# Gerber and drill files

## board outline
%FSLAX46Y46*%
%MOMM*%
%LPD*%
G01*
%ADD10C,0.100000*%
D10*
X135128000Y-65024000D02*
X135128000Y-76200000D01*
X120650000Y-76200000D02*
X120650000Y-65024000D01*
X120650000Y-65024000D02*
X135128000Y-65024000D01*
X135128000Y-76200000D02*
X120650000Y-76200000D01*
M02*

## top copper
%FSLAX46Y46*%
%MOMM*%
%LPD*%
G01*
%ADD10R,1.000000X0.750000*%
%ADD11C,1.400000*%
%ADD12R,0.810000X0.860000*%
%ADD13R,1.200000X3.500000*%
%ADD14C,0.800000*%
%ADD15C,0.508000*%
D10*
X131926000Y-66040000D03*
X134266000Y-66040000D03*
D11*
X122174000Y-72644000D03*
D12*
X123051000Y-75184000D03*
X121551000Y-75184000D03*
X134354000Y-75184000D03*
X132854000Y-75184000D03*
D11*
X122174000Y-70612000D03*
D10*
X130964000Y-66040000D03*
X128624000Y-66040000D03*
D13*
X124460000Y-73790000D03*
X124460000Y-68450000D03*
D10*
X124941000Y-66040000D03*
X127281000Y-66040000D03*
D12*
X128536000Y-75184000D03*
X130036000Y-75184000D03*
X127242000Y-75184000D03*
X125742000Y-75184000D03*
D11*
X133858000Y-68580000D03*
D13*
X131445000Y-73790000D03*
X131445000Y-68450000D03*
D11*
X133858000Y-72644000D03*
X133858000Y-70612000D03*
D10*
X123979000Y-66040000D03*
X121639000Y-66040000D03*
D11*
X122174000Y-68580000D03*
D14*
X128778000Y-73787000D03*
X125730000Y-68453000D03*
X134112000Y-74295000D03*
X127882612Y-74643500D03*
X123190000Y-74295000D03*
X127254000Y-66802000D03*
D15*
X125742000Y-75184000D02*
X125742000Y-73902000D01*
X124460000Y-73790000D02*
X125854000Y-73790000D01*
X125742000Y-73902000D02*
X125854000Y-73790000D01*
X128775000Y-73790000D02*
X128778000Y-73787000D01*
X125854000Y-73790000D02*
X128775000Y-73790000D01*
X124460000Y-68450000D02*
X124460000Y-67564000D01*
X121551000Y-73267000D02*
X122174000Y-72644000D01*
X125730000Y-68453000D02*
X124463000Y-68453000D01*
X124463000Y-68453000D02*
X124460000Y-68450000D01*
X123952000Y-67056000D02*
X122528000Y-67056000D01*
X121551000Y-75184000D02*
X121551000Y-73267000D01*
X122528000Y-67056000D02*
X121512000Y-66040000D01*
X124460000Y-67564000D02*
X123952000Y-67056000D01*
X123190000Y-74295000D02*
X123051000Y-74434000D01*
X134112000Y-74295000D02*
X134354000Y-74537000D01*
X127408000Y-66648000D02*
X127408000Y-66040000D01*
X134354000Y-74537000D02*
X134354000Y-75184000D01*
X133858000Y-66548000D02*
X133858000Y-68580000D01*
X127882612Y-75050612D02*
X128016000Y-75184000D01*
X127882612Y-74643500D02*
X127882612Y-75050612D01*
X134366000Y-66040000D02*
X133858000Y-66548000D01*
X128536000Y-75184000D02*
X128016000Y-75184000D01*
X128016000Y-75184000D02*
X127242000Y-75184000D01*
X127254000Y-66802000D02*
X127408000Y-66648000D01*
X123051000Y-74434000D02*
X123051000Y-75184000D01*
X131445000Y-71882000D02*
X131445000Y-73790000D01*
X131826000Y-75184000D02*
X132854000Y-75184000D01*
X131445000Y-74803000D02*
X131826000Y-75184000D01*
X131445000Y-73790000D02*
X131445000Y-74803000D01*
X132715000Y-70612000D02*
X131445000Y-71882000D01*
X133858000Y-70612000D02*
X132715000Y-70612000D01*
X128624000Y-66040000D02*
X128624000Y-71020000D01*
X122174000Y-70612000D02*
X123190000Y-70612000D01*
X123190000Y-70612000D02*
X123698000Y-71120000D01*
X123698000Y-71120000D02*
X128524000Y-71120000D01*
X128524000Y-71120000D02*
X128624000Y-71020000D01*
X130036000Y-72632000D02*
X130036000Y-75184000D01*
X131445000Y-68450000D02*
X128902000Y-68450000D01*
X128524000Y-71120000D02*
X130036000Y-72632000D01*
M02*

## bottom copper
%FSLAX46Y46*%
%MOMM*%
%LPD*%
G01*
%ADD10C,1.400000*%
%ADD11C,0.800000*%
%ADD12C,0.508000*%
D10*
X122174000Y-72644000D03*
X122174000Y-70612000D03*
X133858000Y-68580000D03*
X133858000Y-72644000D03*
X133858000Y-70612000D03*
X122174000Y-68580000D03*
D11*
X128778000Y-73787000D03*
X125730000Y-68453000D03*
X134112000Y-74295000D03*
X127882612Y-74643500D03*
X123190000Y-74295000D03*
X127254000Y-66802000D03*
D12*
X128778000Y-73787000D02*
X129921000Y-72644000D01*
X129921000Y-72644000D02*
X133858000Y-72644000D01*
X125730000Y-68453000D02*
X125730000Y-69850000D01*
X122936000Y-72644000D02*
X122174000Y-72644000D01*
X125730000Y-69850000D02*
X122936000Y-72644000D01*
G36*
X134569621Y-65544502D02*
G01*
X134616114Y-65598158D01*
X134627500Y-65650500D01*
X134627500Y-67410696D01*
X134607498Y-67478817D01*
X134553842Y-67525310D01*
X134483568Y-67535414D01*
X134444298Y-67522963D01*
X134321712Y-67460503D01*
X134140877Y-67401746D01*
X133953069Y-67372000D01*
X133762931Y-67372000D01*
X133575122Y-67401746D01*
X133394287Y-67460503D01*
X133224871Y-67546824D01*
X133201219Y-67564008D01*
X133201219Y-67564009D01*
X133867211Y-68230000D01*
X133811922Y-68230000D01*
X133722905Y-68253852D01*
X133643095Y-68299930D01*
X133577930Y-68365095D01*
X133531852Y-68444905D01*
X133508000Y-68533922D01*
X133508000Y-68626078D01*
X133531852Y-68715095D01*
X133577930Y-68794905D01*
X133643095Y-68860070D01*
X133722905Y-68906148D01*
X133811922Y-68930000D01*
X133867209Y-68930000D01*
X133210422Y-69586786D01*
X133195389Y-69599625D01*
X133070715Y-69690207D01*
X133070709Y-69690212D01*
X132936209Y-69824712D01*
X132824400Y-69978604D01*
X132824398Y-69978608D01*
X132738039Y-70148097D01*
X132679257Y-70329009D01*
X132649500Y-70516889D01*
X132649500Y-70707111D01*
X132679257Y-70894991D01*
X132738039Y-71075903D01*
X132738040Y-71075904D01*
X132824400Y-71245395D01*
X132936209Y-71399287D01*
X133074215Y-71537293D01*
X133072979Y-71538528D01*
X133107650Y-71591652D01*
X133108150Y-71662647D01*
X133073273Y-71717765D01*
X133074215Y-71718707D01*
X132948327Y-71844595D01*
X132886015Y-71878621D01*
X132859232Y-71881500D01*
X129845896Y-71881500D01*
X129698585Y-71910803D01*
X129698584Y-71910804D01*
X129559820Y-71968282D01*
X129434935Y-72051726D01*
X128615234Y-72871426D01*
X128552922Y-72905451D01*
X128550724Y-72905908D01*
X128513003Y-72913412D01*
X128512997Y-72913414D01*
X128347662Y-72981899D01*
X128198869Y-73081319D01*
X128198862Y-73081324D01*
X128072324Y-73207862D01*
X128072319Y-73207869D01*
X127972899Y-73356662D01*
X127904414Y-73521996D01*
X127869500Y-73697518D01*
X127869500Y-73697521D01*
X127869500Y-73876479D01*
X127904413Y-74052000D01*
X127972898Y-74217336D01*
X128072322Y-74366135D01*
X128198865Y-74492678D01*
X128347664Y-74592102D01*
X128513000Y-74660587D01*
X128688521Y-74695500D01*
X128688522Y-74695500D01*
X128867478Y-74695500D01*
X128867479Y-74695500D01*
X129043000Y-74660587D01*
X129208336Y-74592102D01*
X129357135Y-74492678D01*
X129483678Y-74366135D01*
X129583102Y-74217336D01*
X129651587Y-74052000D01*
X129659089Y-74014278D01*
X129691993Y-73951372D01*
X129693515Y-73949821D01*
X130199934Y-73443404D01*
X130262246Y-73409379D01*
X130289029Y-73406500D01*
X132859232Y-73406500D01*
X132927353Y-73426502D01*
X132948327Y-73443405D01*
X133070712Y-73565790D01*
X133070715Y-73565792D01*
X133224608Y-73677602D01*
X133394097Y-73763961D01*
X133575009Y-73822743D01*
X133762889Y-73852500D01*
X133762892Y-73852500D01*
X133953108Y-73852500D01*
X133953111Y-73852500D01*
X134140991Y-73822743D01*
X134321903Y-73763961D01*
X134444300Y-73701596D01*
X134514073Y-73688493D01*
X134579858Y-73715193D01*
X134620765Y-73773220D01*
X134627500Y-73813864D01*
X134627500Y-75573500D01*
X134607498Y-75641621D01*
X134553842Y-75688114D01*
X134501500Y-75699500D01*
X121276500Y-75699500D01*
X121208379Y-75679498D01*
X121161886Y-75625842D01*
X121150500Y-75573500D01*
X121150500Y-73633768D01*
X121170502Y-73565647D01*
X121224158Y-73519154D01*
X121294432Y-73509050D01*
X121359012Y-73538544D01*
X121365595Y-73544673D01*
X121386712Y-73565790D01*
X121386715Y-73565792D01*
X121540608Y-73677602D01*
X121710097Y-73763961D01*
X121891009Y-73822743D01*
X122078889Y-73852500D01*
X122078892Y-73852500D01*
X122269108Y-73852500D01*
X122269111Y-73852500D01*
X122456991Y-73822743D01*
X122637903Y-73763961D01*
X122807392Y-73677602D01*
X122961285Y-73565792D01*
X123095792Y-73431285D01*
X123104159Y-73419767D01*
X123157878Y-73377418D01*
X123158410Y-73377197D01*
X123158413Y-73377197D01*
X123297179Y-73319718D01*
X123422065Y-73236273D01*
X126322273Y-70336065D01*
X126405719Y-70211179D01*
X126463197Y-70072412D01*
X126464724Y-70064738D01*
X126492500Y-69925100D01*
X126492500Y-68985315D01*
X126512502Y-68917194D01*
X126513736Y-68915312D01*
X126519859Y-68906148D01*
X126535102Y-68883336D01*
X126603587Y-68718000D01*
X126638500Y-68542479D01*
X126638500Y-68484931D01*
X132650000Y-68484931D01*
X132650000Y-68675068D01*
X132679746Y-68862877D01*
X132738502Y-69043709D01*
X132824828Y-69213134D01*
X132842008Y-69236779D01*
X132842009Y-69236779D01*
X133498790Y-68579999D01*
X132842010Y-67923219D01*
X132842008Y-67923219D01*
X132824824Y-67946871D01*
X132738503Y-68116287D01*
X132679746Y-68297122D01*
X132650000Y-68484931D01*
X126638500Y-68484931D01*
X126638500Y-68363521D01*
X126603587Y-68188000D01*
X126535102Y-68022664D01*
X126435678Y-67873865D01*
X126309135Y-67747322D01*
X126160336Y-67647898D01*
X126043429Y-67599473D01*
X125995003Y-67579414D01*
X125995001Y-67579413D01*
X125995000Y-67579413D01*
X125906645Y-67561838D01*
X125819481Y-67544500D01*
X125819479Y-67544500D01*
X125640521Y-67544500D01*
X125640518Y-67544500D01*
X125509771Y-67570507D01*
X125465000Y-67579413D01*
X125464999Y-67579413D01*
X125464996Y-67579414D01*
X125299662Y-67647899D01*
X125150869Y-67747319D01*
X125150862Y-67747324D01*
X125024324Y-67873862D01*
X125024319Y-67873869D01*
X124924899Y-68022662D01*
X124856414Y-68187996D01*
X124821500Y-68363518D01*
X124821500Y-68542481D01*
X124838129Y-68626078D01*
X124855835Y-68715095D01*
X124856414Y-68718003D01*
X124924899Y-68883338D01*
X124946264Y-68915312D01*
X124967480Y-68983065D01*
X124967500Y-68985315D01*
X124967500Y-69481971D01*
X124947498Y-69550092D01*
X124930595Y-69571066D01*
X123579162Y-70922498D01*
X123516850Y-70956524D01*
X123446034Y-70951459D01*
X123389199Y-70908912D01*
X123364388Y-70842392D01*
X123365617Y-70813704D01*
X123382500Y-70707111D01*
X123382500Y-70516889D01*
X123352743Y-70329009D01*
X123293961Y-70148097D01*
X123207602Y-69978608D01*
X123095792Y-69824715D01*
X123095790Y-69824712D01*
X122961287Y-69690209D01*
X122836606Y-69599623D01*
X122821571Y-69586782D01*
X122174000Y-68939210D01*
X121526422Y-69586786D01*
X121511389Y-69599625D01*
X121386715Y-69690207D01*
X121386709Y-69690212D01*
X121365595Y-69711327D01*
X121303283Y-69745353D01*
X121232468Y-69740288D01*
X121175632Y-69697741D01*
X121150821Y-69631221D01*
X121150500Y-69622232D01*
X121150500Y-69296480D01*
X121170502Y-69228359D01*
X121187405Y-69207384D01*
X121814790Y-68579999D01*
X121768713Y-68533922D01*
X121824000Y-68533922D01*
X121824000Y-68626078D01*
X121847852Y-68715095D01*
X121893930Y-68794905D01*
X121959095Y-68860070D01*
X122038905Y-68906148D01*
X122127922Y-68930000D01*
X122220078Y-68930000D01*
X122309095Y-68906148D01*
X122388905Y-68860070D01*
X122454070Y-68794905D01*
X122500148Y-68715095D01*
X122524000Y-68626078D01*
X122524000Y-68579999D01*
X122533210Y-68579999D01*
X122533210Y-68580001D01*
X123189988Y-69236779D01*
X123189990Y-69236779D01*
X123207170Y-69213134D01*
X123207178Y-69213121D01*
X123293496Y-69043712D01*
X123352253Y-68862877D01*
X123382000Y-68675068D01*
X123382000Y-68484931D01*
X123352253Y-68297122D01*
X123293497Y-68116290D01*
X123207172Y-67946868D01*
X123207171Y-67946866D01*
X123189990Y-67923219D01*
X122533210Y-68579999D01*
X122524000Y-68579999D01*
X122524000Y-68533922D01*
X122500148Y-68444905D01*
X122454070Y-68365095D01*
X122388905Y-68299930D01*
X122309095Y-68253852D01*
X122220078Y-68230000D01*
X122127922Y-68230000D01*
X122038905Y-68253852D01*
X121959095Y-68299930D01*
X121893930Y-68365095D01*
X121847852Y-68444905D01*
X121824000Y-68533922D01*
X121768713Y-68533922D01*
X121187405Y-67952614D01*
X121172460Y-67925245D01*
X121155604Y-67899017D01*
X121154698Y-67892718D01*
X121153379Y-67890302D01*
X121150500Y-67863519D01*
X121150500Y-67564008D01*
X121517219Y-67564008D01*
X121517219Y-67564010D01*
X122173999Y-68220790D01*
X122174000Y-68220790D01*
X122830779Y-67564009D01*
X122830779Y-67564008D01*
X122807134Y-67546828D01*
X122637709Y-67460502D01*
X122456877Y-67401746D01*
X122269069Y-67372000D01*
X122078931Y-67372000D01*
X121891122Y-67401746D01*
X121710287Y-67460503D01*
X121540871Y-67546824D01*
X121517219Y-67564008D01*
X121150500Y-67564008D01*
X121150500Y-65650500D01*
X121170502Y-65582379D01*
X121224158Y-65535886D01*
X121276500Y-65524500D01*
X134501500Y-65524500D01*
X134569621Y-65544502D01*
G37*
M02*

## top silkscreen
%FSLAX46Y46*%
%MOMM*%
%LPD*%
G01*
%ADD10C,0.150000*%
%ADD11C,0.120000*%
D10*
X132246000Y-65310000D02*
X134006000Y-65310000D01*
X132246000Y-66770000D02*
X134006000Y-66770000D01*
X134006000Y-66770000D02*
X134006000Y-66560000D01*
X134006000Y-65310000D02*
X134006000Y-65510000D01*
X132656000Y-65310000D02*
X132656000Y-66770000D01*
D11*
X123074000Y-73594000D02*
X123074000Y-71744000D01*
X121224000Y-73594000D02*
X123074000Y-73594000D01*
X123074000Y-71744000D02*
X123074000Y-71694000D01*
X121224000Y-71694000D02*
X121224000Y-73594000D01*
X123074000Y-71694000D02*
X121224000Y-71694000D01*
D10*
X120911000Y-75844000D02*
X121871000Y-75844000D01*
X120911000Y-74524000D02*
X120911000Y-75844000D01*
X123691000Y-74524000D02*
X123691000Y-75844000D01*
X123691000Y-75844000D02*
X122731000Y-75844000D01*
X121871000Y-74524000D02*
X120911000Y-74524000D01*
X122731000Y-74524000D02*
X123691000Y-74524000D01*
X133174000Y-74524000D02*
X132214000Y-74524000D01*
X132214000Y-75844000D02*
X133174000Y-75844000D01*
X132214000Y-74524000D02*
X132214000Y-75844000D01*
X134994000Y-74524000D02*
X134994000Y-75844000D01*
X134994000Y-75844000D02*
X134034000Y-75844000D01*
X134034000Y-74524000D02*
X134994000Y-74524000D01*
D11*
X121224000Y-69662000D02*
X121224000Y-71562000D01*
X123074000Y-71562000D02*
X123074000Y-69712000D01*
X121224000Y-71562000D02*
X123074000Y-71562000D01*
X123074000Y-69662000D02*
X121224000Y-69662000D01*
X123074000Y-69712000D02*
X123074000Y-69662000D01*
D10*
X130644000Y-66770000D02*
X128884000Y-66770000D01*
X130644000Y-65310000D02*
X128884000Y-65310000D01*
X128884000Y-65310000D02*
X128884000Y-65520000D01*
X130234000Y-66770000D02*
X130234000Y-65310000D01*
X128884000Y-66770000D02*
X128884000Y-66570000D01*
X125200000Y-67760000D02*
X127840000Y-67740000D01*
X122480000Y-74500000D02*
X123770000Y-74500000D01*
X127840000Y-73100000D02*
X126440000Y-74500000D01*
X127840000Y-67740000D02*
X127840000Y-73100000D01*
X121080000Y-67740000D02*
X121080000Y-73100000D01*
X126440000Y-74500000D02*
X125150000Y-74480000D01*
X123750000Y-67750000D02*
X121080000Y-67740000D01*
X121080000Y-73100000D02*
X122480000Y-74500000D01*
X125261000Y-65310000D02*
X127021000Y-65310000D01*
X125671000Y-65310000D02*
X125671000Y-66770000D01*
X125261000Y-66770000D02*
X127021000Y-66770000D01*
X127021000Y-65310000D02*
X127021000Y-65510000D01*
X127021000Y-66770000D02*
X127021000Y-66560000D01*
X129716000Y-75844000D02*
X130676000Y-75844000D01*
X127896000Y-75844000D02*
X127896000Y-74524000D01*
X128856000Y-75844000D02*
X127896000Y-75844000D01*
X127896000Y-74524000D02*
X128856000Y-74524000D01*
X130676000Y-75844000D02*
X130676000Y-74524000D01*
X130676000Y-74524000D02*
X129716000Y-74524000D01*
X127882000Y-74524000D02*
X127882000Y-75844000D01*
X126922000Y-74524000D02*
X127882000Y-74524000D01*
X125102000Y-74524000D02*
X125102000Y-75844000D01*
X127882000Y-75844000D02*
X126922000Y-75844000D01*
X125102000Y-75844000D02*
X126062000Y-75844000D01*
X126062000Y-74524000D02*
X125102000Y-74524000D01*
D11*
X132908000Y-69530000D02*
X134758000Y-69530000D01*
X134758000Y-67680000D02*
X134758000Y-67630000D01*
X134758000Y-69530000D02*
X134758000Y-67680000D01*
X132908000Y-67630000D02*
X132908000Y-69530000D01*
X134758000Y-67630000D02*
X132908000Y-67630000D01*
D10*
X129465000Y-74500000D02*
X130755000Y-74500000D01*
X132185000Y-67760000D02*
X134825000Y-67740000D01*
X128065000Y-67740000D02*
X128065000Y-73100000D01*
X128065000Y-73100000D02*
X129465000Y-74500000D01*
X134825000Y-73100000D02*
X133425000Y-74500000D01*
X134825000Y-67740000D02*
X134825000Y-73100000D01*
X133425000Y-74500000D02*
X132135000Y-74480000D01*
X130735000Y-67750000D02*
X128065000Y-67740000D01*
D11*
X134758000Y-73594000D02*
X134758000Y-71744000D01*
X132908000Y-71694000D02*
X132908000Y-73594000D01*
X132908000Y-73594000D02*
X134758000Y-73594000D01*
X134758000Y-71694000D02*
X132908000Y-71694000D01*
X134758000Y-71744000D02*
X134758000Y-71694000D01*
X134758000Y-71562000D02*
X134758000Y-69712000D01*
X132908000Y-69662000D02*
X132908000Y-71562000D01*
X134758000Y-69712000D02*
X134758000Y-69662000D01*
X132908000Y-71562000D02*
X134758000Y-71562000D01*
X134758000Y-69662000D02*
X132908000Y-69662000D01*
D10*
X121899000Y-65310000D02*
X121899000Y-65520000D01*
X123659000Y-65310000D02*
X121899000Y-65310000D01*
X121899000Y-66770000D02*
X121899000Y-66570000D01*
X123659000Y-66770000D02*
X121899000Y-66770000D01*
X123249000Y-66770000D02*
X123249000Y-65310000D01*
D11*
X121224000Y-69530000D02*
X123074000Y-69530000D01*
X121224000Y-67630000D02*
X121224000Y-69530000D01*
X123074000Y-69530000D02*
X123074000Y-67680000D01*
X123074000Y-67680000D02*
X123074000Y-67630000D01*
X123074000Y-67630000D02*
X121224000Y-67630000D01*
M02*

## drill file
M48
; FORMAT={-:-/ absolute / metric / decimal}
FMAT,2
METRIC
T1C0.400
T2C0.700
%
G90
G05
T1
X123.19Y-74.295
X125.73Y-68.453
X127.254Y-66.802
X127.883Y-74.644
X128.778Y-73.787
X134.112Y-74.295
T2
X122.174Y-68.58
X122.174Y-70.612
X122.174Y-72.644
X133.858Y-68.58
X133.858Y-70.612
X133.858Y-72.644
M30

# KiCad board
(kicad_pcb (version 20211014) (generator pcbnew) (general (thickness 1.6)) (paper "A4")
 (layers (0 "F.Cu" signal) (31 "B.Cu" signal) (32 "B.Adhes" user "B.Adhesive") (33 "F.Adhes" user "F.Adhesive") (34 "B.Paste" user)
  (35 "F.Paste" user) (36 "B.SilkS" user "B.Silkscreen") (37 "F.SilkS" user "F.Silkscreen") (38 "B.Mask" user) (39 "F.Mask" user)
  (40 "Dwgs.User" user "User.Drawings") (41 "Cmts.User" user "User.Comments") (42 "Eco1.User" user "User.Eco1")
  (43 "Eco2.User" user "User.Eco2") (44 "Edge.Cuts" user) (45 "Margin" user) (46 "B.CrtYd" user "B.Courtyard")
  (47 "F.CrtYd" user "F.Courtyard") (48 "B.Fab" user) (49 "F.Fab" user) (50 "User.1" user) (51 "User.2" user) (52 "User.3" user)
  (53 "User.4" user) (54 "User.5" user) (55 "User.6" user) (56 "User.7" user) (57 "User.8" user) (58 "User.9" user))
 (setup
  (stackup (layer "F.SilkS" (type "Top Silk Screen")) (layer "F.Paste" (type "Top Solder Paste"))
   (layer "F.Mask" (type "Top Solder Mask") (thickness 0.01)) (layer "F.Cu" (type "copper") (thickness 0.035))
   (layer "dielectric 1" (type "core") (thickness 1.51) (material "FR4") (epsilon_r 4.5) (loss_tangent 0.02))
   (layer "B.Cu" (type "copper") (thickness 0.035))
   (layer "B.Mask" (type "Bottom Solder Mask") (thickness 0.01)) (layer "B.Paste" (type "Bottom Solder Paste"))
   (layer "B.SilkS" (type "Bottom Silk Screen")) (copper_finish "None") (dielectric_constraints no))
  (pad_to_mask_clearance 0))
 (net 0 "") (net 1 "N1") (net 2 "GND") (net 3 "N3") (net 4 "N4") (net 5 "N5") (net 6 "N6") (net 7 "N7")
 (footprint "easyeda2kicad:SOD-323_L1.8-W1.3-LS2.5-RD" (layer "F.Cu") (at 133.096 66.04)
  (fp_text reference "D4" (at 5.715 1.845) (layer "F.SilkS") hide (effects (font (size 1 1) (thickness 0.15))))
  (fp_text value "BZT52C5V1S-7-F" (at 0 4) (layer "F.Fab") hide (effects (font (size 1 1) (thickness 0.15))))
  (fp_line (start -0.85 -0.73) (end 0.91 -0.73) (layer "F.SilkS") (width 0.15))
  (fp_line (start -0.85 0.73) (end 0.91 0.73) (layer "F.SilkS") (width 0.15))
  (fp_line (start 0.91 0.73) (end 0.91 0.52) (layer "F.SilkS") (width 0.15))
  (fp_line (start 0.91 -0.73) (end 0.91 -0.53) (layer "F.SilkS") (width 0.15))
  (fp_line (start -0.44 -0.73) (end -0.44 0.73) (layer "F.SilkS") (width 0.15))
  (pad "1" smd rect locked (at -1.17 0) (size 1 0.75) (layers "F.Cu" "F.Paste" "F.Mask") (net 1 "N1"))
  (pad "2" smd rect locked (at 1.17 0) (size 1 0.75) (layers "F.Cu" "F.Paste" "F.Mask") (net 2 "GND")))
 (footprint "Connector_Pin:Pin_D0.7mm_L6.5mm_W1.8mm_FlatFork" (layer "F.Cu") (at 122.174 72.644)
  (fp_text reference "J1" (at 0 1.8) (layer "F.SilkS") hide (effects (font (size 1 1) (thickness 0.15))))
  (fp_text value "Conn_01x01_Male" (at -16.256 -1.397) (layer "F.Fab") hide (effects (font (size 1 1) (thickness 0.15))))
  (fp_line (start 0.9 0.95) (end 0.9 -0.9) (layer "F.SilkS") (width 0.12))
  (fp_line (start -0.95 0.95) (end 0.9 0.95) (layer "F.SilkS") (width 0.12))
  (fp_line (start 0.9 -0.9) (end 0.9 -0.95) (layer "F.SilkS") (width 0.12))
  (fp_line (start -0.95 -0.95) (end -0.95 0.95) (layer "F.SilkS") (width 0.12))
  (fp_line (start 0.9 -0.95) (end -0.95 -0.95) (layer "F.SilkS") (width 0.12))
  (pad "1" thru_hole circle (at 0 0) (size 1.4 1.4) (drill 0.7) (layers *.Cu *.Mask) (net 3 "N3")))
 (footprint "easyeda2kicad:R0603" (layer "F.Cu") (at 122.301 75.184 180)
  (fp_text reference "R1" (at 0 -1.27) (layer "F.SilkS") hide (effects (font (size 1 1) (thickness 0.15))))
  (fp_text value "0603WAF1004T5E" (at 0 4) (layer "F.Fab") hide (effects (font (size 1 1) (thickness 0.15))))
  (fp_line (start 1.39 -0.66) (end 0.43 -0.66) (layer "F.SilkS") (width 0.15))
  (fp_line (start 1.39 0.66) (end 1.39 -0.66) (layer "F.SilkS") (width 0.15))
  (fp_line (start -1.39 0.66) (end -1.39 -0.66) (layer "F.SilkS") (width 0.15))
  (fp_line (start -1.39 -0.66) (end -0.43 -0.66) (layer "F.SilkS") (width 0.15))
  (fp_line (start 0.43 0.66) (end 1.39 0.66) (layer "F.SilkS") (width 0.15))
  (fp_line (start -0.43 0.66) (end -1.39 0.66) (layer "F.SilkS") (width 0.15))
  (pad "1" smd rect locked (at -0.75 0 180) (size 0.81 0.86) (layers "F.Cu" "F.Paste" "F.Mask") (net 2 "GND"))
  (pad "2" smd rect locked (at 0.75 0 180) (size 0.81 0.86) (layers "F.Cu" "F.Paste" "F.Mask") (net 3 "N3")))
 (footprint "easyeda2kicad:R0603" (layer "F.Cu") (at 133.604 75.184 180)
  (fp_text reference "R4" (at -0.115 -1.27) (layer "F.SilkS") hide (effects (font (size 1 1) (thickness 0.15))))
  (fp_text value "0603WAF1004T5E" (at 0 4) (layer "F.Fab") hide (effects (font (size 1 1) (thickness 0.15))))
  (fp_line (start 0.43 0.66) (end 1.39 0.66) (layer "F.SilkS") (width 0.15))
  (fp_line (start 1.39 -0.66) (end 0.43 -0.66) (layer "F.SilkS") (width 0.15))
  (fp_line (start 1.39 0.66) (end 1.39 -0.66) (layer "F.SilkS") (width 0.15))
  (fp_line (start -1.39 0.66) (end -1.39 -0.66) (layer "F.SilkS") (width 0.15))
  (fp_line (start -1.39 -0.66) (end -0.43 -0.66) (layer "F.SilkS") (width 0.15))
  (fp_line (start -0.43 0.66) (end -1.39 0.66) (layer "F.SilkS") (width 0.15))
  (pad "1" smd rect locked (at -0.75 0 180) (size 0.81 0.86) (layers "F.Cu" "F.Paste" "F.Mask") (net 2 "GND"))
  (pad "2" smd rect locked (at 0.75 0 180) (size 0.81 0.86) (layers "F.Cu" "F.Paste" "F.Mask") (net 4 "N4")))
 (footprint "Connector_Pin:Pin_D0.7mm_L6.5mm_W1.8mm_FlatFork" (layer "F.Cu") (at 122.174 70.612)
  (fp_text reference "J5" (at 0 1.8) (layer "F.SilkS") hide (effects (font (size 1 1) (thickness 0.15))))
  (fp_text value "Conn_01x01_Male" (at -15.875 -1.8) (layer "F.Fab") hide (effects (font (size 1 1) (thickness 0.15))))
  (fp_line (start -0.95 -0.95) (end -0.95 0.95) (layer "F.SilkS") (width 0.12))
  (fp_line (start 0.9 0.95) (end 0.9 -0.9) (layer "F.SilkS") (width 0.12))
  (fp_line (start -0.95 0.95) (end 0.9 0.95) (layer "F.SilkS") (width 0.12))
  (fp_line (start 0.9 -0.95) (end -0.95 -0.95) (layer "F.SilkS") (width 0.12))
  (fp_line (start 0.9 -0.9) (end 0.9 -0.95) (layer "F.SilkS") (width 0.12))
  (pad "1" thru_hole circle (at 0 0) (size 1.4 1.4) (drill 0.7) (layers *.Cu *.Mask) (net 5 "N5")))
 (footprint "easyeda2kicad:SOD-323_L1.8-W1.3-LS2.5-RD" (layer "F.Cu") (at 129.794 66.04 180)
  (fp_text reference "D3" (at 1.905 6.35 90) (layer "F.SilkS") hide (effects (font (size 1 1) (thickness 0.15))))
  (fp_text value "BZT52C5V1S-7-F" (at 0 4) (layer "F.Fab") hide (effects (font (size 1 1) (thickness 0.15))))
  (fp_line (start -0.85 -0.73) (end 0.91 -0.73) (layer "F.SilkS") (width 0.15))
  (fp_line (start -0.85 0.73) (end 0.91 0.73) (layer "F.SilkS") (width 0.15))
  (fp_line (start 0.91 0.73) (end 0.91 0.52) (layer "F.SilkS") (width 0.15))
  (fp_line (start -0.44 -0.73) (end -0.44 0.73) (layer "F.SilkS") (width 0.15))
  (fp_line (start 0.91 -0.73) (end 0.91 -0.53) (layer "F.SilkS") (width 0.15))
  (pad "1" smd rect locked (at -1.17 0 180) (size 1 0.75) (layers "F.Cu" "F.Paste" "F.Mask") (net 1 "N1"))
  (pad "2" smd rect locked (at 1.17 0 180) (size 1 0.75) (layers "F.Cu" "F.Paste" "F.Mask") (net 5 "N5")))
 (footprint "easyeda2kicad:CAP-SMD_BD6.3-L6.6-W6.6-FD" (layer "F.Cu") (at 124.46 71.12 90)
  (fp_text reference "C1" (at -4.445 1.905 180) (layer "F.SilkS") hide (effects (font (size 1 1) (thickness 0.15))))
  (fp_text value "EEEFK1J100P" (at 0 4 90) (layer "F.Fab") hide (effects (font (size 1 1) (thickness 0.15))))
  (fp_line (start 3.36 0.74) (end 3.38 3.38) (layer "F.SilkS") (width 0.15))
  (fp_line (start -3.38 -1.98) (end -3.38 -0.69) (layer "F.SilkS") (width 0.15))
  (fp_line (start -1.98 3.38) (end -3.38 1.98) (layer "F.SilkS") (width 0.15))
  (fp_line (start 3.38 3.38) (end -1.98 3.38) (layer "F.SilkS") (width 0.15))
  (fp_line (start 3.38 -3.38) (end -1.98 -3.38) (layer "F.SilkS") (width 0.15))
  (fp_line (start -3.38 1.98) (end -3.36 0.69) (layer "F.SilkS") (width 0.15))
  (fp_line (start 3.37 -0.71) (end 3.38 -3.38) (layer "F.SilkS") (width 0.15))
  (fp_line (start -1.98 -3.38) (end -3.38 -1.98) (layer "F.SilkS") (width 0.15))
  (pad "1" smd rect locked (at -2.67 0 90) (size 3.5 1.2) (layers "F.Cu" "F.Paste" "F.Mask") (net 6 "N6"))
  (pad "2" smd rect locked (at 2.67 0 90) (size 3.5 1.2) (layers "F.Cu" "F.Paste" "F.Mask") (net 3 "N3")))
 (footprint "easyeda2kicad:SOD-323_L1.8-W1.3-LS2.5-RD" (layer "F.Cu") (at 126.111 66.04)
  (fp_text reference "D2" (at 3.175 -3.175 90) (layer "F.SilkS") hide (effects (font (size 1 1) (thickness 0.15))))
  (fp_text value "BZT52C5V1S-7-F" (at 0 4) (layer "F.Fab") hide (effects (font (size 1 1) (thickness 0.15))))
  (fp_line (start -0.85 -0.73) (end 0.91 -0.73) (layer "F.SilkS") (width 0.15))
  (fp_line (start -0.44 -0.73) (end -0.44 0.73) (layer "F.SilkS") (width 0.15))
  (fp_line (start -0.85 0.73) (end 0.91 0.73) (layer "F.SilkS") (width 0.15))
  (fp_line (start 0.91 -0.73) (end 0.91 -0.53) (layer "F.SilkS") (width 0.15))
  (fp_line (start 0.91 0.73) (end 0.91 0.52) (layer "F.SilkS") (width 0.15))
  (pad "1" smd rect locked (at -1.17 0) (size 1 0.75) (layers "F.Cu" "F.Paste" "F.Mask") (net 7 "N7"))
  (pad "2" smd rect locked (at 1.17 0) (size 1 0.75) (layers "F.Cu" "F.Paste" "F.Mask") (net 2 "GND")))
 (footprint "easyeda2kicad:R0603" (layer "F.Cu") (at 129.286 75.184)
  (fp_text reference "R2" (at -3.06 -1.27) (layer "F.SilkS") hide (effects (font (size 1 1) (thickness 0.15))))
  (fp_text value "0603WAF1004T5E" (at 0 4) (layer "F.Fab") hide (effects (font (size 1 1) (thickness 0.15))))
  (fp_line (start 0.43 0.66) (end 1.39 0.66) (layer "F.SilkS") (width 0.15))
  (fp_line (start -1.39 0.66) (end -1.39 -0.66) (layer "F.SilkS") (width 0.15))
  (fp_line (start -0.43 0.66) (end -1.39 0.66) (layer "F.SilkS") (width 0.15))
  (fp_line (start -1.39 -0.66) (end -0.43 -0.66) (layer "F.SilkS") (width 0.15))
  (fp_line (start 1.39 0.66) (end 1.39 -0.66) (layer "F.SilkS") (width 0.15))
  (fp_line (start 1.39 -0.66) (end 0.43 -0.66) (layer "F.SilkS") (width 0.15))
  (pad "1" smd rect locked (at -0.75 0) (size 0.81 0.86) (layers "F.Cu" "F.Paste" "F.Mask") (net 2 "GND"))
  (pad "2" smd rect locked (at 0.75 0) (size 0.81 0.86) (layers "F.Cu" "F.Paste" "F.Mask") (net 5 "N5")))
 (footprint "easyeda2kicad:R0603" (layer "F.Cu") (at 126.492 75.184 180)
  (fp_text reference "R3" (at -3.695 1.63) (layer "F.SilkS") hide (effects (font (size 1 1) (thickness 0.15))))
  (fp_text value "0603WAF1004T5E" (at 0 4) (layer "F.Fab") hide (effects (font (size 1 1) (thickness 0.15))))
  (fp_line (start -1.39 0.66) (end -1.39 -0.66) (layer "F.SilkS") (width 0.15))
  (fp_line (start -0.43 0.66) (end -1.39 0.66) (layer "F.SilkS") (width 0.15))
  (fp_line (start 1.39 0.66) (end 1.39 -0.66) (layer "F.SilkS") (width 0.15))
  (fp_line (start -1.39 -0.66) (end -0.43 -0.66) (layer "F.SilkS") (width 0.15))
  (fp_line (start 1.39 -0.66) (end 0.43 -0.66) (layer "F.SilkS") (width 0.15))
  (fp_line (start 0.43 0.66) (end 1.39 0.66) (layer "F.SilkS") (width 0.15))
  (pad "1" smd rect locked (at -0.75 0 180) (size 0.81 0.86) (layers "F.Cu" "F.Paste" "F.Mask") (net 2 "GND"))
  (pad "2" smd rect locked (at 0.75 0 180) (size 0.81 0.86) (layers "F.Cu" "F.Paste" "F.Mask") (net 6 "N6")))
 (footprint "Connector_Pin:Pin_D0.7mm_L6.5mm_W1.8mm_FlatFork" (layer "F.Cu") (at 133.858 68.58)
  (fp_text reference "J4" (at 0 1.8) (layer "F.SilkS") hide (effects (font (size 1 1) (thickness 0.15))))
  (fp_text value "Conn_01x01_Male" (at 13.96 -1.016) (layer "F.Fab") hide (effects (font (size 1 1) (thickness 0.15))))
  (fp_line (start -0.95 0.95) (end 0.9 0.95) (layer "F.SilkS") (width 0.12))
  (fp_line (start 0.9 -0.9) (end 0.9 -0.95) (layer "F.SilkS") (width 0.12))
  (fp_line (start 0.9 0.95) (end 0.9 -0.9) (layer "F.SilkS") (width 0.12))
  (fp_line (start -0.95 -0.95) (end -0.95 0.95) (layer "F.SilkS") (width 0.12))
  (fp_line (start 0.9 -0.95) (end -0.95 -0.95) (layer "F.SilkS") (width 0.12))
  (pad "1" thru_hole circle (at 0 0) (size 1.4 1.4) (drill 0.7) (layers *.Cu *.Mask) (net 2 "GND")))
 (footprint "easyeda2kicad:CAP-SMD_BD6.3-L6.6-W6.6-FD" (layer "F.Cu") (at 131.445 71.12 90)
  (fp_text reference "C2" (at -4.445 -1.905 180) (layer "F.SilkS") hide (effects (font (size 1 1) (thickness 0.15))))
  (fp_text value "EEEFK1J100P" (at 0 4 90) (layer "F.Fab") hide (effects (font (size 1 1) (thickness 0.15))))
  (fp_line (start -3.38 -1.98) (end -3.38 -0.69) (layer "F.SilkS") (width 0.15))
  (fp_line (start 3.36 0.74) (end 3.38 3.38) (layer "F.SilkS") (width 0.15))
  (fp_line (start 3.38 -3.38) (end -1.98 -3.38) (layer "F.SilkS") (width 0.15))
  (fp_line (start -1.98 -3.38) (end -3.38 -1.98) (layer "F.SilkS") (width 0.15))
  (fp_line (start -1.98 3.38) (end -3.38 1.98) (layer "F.SilkS") (width 0.15))
  (fp_line (start 3.38 3.38) (end -1.98 3.38) (layer "F.SilkS") (width 0.15))
  (fp_line (start -3.38 1.98) (end -3.36 0.69) (layer "F.SilkS") (width 0.15))
  (fp_line (start 3.37 -0.71) (end 3.38 -3.38) (layer "F.SilkS") (width 0.15))
  (pad "1" smd rect locked (at -2.67 0 90) (size 3.5 1.2) (layers "F.Cu" "F.Paste" "F.Mask") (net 4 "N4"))
  (pad "2" smd rect locked (at 2.67 0 90) (size 3.5 1.2) (layers "F.Cu" "F.Paste" "F.Mask") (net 5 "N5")))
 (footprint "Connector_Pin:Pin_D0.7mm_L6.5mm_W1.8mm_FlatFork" (layer "F.Cu") (at 133.858 72.644)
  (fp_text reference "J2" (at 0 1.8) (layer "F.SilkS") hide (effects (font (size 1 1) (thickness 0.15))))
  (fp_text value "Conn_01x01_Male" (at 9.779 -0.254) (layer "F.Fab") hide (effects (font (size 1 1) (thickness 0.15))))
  (fp_line (start 0.9 0.95) (end 0.9 -0.9) (layer "F.SilkS") (width 0.12))
  (fp_line (start -0.95 -0.95) (end -0.95 0.95) (layer "F.SilkS") (width 0.12))
  (fp_line (start -0.95 0.95) (end 0.9 0.95) (layer "F.SilkS") (width 0.12))
  (fp_line (start 0.9 -0.95) (end -0.95 -0.95) (layer "F.SilkS") (width 0.12))
  (fp_line (start 0.9 -0.9) (end 0.9 -0.95) (layer "F.SilkS") (width 0.12))
  (pad "1" thru_hole circle (at 0 0) (size 1.4 1.4) (drill 0.7) (layers *.Cu *.Mask) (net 6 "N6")))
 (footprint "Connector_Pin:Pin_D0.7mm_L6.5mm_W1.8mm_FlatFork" (layer "F.Cu") (at 133.858 70.612)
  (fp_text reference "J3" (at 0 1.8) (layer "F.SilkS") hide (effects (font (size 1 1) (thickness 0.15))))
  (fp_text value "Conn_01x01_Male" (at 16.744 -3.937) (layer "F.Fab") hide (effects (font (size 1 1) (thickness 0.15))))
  (fp_line (start 0.9 0.95) (end 0.9 -0.9) (layer "F.SilkS") (width 0.12))
  (fp_line (start -0.95 -0.95) (end -0.95 0.95) (layer "F.SilkS") (width 0.12))
  (fp_line (start 0.9 -0.9) (end 0.9 -0.95) (layer "F.SilkS") (width 0.12))
  (fp_line (start -0.95 0.95) (end 0.9 0.95) (layer "F.SilkS") (width 0.12))
  (fp_line (start 0.9 -0.95) (end -0.95 -0.95) (layer "F.SilkS") (width 0.12))
  (pad "1" thru_hole circle (at 0 0) (size 1.4 1.4) (drill 0.7) (layers *.Cu *.Mask) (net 4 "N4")))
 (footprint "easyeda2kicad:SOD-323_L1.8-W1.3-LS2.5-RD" (layer "F.Cu") (at 122.809 66.04 180)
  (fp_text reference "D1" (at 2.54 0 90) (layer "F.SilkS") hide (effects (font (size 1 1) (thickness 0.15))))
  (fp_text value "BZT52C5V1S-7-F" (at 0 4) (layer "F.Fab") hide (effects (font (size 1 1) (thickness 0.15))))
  (fp_line (start 0.91 0.73) (end 0.91 0.52) (layer "F.SilkS") (width 0.15))
  (fp_line (start -0.85 0.73) (end 0.91 0.73) (layer "F.SilkS") (width 0.15))
  (fp_line (start 0.91 -0.73) (end 0.91 -0.53) (layer "F.SilkS") (width 0.15))
  (fp_line (start -0.85 -0.73) (end 0.91 -0.73) (layer "F.SilkS") (width 0.15))
  (fp_line (start -0.44 -0.73) (end -0.44 0.73) (layer "F.SilkS") (width 0.15))
  (pad "1" smd rect locked (at -1.17 0 180) (size 1 0.75) (layers "F.Cu" "F.Paste" "F.Mask") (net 7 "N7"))
  (pad "2" smd rect locked (at 1.17 0 180) (size 1 0.75) (layers "F.Cu" "F.Paste" "F.Mask") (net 3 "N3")))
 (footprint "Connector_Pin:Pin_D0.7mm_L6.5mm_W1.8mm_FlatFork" (layer "F.Cu") (at 122.174 68.58)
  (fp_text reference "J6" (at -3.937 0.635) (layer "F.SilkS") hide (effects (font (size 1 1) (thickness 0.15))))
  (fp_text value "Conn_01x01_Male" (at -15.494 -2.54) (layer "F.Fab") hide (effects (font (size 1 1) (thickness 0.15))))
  (fp_line (start -0.95 0.95) (end 0.9 0.95) (layer "F.SilkS") (width 0.12))
  (fp_line (start -0.95 -0.95) (end -0.95 0.95) (layer "F.SilkS") (width 0.12))
  (fp_line (start 0.9 0.95) (end 0.9 -0.9) (layer "F.SilkS") (width 0.12))
  (fp_line (start 0.9 -0.9) (end 0.9 -0.95) (layer "F.SilkS") (width 0.12))
  (fp_line (start 0.9 -0.95) (end -0.95 -0.95) (layer "F.SilkS") (width 0.12))
  (pad "1" thru_hole circle (at 0 0) (size 1.4 1.4) (drill 0.7) (layers *.Cu *.Mask) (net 2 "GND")))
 (gr_line (start 135.128 65.024) (end 135.128 76.2) (layer "Edge.Cuts") (width 0.1))
 (gr_line (start 120.65 76.2) (end 120.65 65.024) (layer "Edge.Cuts") (width 0.1))
 (gr_line (start 120.65 65.024) (end 135.128 65.024) (layer "Edge.Cuts") (width 0.1))
 (gr_line (start 135.128 76.2) (end 120.65 76.2) (layer "Edge.Cuts") (width 0.1))
 (segment (start 125.742 75.184) (end 125.742 73.902) (width 0.508) (layer "F.Cu") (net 6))
 (segment (start 124.46 73.79) (end 125.854 73.79) (width 0.508) (layer "F.Cu") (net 6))
 (segment (start 125.742 73.902) (end 125.854 73.79) (width 0.508) (layer "F.Cu") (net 6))
 (segment (start 128.775 73.79) (end 128.778 73.787) (width 0.508) (layer "F.Cu") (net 6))
 (segment (start 125.854 73.79) (end 128.775 73.79) (width 0.508) (layer "F.Cu") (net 6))
 (via (at 128.778 73.787) (size 0.8) (drill 0.4) (layers "F.Cu" "B.Cu") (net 6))
 (segment (start 128.778 73.787) (end 129.921 72.644) (width 0.508) (layer "B.Cu") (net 6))
 (segment (start 129.921 72.644) (end 133.858 72.644) (width 0.508) (layer "B.Cu") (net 6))
 (segment (start 124.46 68.45) (end 124.46 67.564) (width 0.508) (layer "F.Cu") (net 3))
 (segment (start 121.551 73.267) (end 122.174 72.644) (width 0.508) (layer "F.Cu") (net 3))
 (segment (start 125.73 68.453) (end 124.463 68.453) (width 0.508) (layer "F.Cu") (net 3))
 (segment (start 124.463 68.453) (end 124.46 68.45) (width 0.508) (layer "F.Cu") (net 3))
 (segment (start 123.952 67.056) (end 122.528 67.056) (width 0.508) (layer "F.Cu") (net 3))
 (segment (start 121.551 75.184) (end 121.551 73.267) (width 0.508) (layer "F.Cu") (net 3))
 (segment (start 122.528 67.056) (end 121.512 66.04) (width 0.508) (layer "F.Cu") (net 3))
 (segment (start 124.46 67.564) (end 123.952 67.056) (width 0.508) (layer "F.Cu") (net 3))
 (via (at 125.73 68.453) (size 0.8) (drill 0.4) (layers "F.Cu" "B.Cu") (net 3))
 (segment (start 125.73 68.453) (end 125.73 69.85) (width 0.508) (layer "B.Cu") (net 3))
 (segment (start 122.936 72.644) (end 122.174 72.644) (width 0.508) (layer "B.Cu") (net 3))
 (segment (start 125.73 69.85) (end 122.936 72.644) (width 0.508) (layer "B.Cu") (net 3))
 (segment (start 123.19 74.295) (end 123.051 74.434) (width 0.508) (layer "F.Cu") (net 2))
 (segment (start 134.112 74.295) (end 134.354 74.537) (width 0.508) (layer "F.Cu") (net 2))
 (segment (start 127.408 66.648) (end 127.408 66.04) (width 0.508) (layer "F.Cu") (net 2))
 (segment (start 134.354 74.537) (end 134.354 75.184) (width 0.508) (layer "F.Cu") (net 2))
 (segment (start 133.858 66.548) (end 133.858 68.58) (width 0.508) (layer "F.Cu") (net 2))
 (segment (start 127.882612 75.050612) (end 128.016 75.184) (width 0.508) (layer "F.Cu") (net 2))
 (segment (start 127.882612 74.6435) (end 127.882612 75.050612) (width 0.508) (layer "F.Cu") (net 2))
 (segment (start 134.366 66.04) (end 133.858 66.548) (width 0.508) (layer "F.Cu") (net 2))
 (segment (start 128.536 75.184) (end 128.016 75.184) (width 0.508) (layer "F.Cu") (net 2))
 (segment (start 128.016 75.184) (end 127.242 75.184) (width 0.508) (layer "F.Cu") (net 2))
 (segment (start 127.254 66.802) (end 127.408 66.648) (width 0.508) (layer "F.Cu") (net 2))
 (segment (start 123.051 74.434) (end 123.051 75.184) (width 0.508) (layer "F.Cu") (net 2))
 (via (at 134.112 74.295) (size 0.8) (drill 0.4) (layers "F.Cu" "B.Cu") (free) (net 2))
 (via (at 127.882612 74.6435) (size 0.8) (drill 0.4) (layers "F.Cu" "B.Cu") (free) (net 2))
 (via (at 123.19 74.295) (size 0.8) (drill 0.4) (layers "F.Cu" "B.Cu") (free) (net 2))
 (via (at 127.254 66.802) (size 0.8) (drill 0.4) (layers "F.Cu" "B.Cu") (free) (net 2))
 (segment (start 131.445 71.882) (end 131.445 73.79) (width 0.508) (layer "F.Cu") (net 4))
 (segment (start 131.826 75.184) (end 132.854 75.184) (width 0.508) (layer "F.Cu") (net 4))
 (segment (start 131.445 74.803) (end 131.826 75.184) (width 0.508) (layer "F.Cu") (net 4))
 (segment (start 131.445 73.79) (end 131.445 74.803) (width 0.508) (layer "F.Cu") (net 4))
 (segment (start 132.715 70.612) (end 131.445 71.882) (width 0.508) (layer "F.Cu") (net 4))
 (segment (start 133.858 70.612) (end 132.715 70.612) (width 0.508) (layer "F.Cu") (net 4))
 (segment (start 128.624 66.04) (end 128.624 71.02) (width 0.508) (layer "F.Cu") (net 5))
 (segment (start 122.174 70.612) (end 123.19 70.612) (width 0.508) (layer "F.Cu") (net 5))
 (segment (start 123.19 70.612) (end 123.698 71.12) (width 0.508) (layer "F.Cu") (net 5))
 (segment (start 123.698 71.12) (end 128.524 71.12) (width 0.508) (layer "F.Cu") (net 5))
 (segment (start 128.524 71.12) (end 128.624 71.02) (width 0.508) (layer "F.Cu") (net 5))
 (segment (start 130.036 72.632) (end 130.036 75.184) (width 0.508) (layer "F.Cu") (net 5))
 (segment (start 131.445 68.45) (end 128.902 68.45) (width 0.508) (layer "F.Cu") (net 5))
 (segment (start 128.524 71.12) (end 130.036 72.632) (width 0.508) (layer "F.Cu") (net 5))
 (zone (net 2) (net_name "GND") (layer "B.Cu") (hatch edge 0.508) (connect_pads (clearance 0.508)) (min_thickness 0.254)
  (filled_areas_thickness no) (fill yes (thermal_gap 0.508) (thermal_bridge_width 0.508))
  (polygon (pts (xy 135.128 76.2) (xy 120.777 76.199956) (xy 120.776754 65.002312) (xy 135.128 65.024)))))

